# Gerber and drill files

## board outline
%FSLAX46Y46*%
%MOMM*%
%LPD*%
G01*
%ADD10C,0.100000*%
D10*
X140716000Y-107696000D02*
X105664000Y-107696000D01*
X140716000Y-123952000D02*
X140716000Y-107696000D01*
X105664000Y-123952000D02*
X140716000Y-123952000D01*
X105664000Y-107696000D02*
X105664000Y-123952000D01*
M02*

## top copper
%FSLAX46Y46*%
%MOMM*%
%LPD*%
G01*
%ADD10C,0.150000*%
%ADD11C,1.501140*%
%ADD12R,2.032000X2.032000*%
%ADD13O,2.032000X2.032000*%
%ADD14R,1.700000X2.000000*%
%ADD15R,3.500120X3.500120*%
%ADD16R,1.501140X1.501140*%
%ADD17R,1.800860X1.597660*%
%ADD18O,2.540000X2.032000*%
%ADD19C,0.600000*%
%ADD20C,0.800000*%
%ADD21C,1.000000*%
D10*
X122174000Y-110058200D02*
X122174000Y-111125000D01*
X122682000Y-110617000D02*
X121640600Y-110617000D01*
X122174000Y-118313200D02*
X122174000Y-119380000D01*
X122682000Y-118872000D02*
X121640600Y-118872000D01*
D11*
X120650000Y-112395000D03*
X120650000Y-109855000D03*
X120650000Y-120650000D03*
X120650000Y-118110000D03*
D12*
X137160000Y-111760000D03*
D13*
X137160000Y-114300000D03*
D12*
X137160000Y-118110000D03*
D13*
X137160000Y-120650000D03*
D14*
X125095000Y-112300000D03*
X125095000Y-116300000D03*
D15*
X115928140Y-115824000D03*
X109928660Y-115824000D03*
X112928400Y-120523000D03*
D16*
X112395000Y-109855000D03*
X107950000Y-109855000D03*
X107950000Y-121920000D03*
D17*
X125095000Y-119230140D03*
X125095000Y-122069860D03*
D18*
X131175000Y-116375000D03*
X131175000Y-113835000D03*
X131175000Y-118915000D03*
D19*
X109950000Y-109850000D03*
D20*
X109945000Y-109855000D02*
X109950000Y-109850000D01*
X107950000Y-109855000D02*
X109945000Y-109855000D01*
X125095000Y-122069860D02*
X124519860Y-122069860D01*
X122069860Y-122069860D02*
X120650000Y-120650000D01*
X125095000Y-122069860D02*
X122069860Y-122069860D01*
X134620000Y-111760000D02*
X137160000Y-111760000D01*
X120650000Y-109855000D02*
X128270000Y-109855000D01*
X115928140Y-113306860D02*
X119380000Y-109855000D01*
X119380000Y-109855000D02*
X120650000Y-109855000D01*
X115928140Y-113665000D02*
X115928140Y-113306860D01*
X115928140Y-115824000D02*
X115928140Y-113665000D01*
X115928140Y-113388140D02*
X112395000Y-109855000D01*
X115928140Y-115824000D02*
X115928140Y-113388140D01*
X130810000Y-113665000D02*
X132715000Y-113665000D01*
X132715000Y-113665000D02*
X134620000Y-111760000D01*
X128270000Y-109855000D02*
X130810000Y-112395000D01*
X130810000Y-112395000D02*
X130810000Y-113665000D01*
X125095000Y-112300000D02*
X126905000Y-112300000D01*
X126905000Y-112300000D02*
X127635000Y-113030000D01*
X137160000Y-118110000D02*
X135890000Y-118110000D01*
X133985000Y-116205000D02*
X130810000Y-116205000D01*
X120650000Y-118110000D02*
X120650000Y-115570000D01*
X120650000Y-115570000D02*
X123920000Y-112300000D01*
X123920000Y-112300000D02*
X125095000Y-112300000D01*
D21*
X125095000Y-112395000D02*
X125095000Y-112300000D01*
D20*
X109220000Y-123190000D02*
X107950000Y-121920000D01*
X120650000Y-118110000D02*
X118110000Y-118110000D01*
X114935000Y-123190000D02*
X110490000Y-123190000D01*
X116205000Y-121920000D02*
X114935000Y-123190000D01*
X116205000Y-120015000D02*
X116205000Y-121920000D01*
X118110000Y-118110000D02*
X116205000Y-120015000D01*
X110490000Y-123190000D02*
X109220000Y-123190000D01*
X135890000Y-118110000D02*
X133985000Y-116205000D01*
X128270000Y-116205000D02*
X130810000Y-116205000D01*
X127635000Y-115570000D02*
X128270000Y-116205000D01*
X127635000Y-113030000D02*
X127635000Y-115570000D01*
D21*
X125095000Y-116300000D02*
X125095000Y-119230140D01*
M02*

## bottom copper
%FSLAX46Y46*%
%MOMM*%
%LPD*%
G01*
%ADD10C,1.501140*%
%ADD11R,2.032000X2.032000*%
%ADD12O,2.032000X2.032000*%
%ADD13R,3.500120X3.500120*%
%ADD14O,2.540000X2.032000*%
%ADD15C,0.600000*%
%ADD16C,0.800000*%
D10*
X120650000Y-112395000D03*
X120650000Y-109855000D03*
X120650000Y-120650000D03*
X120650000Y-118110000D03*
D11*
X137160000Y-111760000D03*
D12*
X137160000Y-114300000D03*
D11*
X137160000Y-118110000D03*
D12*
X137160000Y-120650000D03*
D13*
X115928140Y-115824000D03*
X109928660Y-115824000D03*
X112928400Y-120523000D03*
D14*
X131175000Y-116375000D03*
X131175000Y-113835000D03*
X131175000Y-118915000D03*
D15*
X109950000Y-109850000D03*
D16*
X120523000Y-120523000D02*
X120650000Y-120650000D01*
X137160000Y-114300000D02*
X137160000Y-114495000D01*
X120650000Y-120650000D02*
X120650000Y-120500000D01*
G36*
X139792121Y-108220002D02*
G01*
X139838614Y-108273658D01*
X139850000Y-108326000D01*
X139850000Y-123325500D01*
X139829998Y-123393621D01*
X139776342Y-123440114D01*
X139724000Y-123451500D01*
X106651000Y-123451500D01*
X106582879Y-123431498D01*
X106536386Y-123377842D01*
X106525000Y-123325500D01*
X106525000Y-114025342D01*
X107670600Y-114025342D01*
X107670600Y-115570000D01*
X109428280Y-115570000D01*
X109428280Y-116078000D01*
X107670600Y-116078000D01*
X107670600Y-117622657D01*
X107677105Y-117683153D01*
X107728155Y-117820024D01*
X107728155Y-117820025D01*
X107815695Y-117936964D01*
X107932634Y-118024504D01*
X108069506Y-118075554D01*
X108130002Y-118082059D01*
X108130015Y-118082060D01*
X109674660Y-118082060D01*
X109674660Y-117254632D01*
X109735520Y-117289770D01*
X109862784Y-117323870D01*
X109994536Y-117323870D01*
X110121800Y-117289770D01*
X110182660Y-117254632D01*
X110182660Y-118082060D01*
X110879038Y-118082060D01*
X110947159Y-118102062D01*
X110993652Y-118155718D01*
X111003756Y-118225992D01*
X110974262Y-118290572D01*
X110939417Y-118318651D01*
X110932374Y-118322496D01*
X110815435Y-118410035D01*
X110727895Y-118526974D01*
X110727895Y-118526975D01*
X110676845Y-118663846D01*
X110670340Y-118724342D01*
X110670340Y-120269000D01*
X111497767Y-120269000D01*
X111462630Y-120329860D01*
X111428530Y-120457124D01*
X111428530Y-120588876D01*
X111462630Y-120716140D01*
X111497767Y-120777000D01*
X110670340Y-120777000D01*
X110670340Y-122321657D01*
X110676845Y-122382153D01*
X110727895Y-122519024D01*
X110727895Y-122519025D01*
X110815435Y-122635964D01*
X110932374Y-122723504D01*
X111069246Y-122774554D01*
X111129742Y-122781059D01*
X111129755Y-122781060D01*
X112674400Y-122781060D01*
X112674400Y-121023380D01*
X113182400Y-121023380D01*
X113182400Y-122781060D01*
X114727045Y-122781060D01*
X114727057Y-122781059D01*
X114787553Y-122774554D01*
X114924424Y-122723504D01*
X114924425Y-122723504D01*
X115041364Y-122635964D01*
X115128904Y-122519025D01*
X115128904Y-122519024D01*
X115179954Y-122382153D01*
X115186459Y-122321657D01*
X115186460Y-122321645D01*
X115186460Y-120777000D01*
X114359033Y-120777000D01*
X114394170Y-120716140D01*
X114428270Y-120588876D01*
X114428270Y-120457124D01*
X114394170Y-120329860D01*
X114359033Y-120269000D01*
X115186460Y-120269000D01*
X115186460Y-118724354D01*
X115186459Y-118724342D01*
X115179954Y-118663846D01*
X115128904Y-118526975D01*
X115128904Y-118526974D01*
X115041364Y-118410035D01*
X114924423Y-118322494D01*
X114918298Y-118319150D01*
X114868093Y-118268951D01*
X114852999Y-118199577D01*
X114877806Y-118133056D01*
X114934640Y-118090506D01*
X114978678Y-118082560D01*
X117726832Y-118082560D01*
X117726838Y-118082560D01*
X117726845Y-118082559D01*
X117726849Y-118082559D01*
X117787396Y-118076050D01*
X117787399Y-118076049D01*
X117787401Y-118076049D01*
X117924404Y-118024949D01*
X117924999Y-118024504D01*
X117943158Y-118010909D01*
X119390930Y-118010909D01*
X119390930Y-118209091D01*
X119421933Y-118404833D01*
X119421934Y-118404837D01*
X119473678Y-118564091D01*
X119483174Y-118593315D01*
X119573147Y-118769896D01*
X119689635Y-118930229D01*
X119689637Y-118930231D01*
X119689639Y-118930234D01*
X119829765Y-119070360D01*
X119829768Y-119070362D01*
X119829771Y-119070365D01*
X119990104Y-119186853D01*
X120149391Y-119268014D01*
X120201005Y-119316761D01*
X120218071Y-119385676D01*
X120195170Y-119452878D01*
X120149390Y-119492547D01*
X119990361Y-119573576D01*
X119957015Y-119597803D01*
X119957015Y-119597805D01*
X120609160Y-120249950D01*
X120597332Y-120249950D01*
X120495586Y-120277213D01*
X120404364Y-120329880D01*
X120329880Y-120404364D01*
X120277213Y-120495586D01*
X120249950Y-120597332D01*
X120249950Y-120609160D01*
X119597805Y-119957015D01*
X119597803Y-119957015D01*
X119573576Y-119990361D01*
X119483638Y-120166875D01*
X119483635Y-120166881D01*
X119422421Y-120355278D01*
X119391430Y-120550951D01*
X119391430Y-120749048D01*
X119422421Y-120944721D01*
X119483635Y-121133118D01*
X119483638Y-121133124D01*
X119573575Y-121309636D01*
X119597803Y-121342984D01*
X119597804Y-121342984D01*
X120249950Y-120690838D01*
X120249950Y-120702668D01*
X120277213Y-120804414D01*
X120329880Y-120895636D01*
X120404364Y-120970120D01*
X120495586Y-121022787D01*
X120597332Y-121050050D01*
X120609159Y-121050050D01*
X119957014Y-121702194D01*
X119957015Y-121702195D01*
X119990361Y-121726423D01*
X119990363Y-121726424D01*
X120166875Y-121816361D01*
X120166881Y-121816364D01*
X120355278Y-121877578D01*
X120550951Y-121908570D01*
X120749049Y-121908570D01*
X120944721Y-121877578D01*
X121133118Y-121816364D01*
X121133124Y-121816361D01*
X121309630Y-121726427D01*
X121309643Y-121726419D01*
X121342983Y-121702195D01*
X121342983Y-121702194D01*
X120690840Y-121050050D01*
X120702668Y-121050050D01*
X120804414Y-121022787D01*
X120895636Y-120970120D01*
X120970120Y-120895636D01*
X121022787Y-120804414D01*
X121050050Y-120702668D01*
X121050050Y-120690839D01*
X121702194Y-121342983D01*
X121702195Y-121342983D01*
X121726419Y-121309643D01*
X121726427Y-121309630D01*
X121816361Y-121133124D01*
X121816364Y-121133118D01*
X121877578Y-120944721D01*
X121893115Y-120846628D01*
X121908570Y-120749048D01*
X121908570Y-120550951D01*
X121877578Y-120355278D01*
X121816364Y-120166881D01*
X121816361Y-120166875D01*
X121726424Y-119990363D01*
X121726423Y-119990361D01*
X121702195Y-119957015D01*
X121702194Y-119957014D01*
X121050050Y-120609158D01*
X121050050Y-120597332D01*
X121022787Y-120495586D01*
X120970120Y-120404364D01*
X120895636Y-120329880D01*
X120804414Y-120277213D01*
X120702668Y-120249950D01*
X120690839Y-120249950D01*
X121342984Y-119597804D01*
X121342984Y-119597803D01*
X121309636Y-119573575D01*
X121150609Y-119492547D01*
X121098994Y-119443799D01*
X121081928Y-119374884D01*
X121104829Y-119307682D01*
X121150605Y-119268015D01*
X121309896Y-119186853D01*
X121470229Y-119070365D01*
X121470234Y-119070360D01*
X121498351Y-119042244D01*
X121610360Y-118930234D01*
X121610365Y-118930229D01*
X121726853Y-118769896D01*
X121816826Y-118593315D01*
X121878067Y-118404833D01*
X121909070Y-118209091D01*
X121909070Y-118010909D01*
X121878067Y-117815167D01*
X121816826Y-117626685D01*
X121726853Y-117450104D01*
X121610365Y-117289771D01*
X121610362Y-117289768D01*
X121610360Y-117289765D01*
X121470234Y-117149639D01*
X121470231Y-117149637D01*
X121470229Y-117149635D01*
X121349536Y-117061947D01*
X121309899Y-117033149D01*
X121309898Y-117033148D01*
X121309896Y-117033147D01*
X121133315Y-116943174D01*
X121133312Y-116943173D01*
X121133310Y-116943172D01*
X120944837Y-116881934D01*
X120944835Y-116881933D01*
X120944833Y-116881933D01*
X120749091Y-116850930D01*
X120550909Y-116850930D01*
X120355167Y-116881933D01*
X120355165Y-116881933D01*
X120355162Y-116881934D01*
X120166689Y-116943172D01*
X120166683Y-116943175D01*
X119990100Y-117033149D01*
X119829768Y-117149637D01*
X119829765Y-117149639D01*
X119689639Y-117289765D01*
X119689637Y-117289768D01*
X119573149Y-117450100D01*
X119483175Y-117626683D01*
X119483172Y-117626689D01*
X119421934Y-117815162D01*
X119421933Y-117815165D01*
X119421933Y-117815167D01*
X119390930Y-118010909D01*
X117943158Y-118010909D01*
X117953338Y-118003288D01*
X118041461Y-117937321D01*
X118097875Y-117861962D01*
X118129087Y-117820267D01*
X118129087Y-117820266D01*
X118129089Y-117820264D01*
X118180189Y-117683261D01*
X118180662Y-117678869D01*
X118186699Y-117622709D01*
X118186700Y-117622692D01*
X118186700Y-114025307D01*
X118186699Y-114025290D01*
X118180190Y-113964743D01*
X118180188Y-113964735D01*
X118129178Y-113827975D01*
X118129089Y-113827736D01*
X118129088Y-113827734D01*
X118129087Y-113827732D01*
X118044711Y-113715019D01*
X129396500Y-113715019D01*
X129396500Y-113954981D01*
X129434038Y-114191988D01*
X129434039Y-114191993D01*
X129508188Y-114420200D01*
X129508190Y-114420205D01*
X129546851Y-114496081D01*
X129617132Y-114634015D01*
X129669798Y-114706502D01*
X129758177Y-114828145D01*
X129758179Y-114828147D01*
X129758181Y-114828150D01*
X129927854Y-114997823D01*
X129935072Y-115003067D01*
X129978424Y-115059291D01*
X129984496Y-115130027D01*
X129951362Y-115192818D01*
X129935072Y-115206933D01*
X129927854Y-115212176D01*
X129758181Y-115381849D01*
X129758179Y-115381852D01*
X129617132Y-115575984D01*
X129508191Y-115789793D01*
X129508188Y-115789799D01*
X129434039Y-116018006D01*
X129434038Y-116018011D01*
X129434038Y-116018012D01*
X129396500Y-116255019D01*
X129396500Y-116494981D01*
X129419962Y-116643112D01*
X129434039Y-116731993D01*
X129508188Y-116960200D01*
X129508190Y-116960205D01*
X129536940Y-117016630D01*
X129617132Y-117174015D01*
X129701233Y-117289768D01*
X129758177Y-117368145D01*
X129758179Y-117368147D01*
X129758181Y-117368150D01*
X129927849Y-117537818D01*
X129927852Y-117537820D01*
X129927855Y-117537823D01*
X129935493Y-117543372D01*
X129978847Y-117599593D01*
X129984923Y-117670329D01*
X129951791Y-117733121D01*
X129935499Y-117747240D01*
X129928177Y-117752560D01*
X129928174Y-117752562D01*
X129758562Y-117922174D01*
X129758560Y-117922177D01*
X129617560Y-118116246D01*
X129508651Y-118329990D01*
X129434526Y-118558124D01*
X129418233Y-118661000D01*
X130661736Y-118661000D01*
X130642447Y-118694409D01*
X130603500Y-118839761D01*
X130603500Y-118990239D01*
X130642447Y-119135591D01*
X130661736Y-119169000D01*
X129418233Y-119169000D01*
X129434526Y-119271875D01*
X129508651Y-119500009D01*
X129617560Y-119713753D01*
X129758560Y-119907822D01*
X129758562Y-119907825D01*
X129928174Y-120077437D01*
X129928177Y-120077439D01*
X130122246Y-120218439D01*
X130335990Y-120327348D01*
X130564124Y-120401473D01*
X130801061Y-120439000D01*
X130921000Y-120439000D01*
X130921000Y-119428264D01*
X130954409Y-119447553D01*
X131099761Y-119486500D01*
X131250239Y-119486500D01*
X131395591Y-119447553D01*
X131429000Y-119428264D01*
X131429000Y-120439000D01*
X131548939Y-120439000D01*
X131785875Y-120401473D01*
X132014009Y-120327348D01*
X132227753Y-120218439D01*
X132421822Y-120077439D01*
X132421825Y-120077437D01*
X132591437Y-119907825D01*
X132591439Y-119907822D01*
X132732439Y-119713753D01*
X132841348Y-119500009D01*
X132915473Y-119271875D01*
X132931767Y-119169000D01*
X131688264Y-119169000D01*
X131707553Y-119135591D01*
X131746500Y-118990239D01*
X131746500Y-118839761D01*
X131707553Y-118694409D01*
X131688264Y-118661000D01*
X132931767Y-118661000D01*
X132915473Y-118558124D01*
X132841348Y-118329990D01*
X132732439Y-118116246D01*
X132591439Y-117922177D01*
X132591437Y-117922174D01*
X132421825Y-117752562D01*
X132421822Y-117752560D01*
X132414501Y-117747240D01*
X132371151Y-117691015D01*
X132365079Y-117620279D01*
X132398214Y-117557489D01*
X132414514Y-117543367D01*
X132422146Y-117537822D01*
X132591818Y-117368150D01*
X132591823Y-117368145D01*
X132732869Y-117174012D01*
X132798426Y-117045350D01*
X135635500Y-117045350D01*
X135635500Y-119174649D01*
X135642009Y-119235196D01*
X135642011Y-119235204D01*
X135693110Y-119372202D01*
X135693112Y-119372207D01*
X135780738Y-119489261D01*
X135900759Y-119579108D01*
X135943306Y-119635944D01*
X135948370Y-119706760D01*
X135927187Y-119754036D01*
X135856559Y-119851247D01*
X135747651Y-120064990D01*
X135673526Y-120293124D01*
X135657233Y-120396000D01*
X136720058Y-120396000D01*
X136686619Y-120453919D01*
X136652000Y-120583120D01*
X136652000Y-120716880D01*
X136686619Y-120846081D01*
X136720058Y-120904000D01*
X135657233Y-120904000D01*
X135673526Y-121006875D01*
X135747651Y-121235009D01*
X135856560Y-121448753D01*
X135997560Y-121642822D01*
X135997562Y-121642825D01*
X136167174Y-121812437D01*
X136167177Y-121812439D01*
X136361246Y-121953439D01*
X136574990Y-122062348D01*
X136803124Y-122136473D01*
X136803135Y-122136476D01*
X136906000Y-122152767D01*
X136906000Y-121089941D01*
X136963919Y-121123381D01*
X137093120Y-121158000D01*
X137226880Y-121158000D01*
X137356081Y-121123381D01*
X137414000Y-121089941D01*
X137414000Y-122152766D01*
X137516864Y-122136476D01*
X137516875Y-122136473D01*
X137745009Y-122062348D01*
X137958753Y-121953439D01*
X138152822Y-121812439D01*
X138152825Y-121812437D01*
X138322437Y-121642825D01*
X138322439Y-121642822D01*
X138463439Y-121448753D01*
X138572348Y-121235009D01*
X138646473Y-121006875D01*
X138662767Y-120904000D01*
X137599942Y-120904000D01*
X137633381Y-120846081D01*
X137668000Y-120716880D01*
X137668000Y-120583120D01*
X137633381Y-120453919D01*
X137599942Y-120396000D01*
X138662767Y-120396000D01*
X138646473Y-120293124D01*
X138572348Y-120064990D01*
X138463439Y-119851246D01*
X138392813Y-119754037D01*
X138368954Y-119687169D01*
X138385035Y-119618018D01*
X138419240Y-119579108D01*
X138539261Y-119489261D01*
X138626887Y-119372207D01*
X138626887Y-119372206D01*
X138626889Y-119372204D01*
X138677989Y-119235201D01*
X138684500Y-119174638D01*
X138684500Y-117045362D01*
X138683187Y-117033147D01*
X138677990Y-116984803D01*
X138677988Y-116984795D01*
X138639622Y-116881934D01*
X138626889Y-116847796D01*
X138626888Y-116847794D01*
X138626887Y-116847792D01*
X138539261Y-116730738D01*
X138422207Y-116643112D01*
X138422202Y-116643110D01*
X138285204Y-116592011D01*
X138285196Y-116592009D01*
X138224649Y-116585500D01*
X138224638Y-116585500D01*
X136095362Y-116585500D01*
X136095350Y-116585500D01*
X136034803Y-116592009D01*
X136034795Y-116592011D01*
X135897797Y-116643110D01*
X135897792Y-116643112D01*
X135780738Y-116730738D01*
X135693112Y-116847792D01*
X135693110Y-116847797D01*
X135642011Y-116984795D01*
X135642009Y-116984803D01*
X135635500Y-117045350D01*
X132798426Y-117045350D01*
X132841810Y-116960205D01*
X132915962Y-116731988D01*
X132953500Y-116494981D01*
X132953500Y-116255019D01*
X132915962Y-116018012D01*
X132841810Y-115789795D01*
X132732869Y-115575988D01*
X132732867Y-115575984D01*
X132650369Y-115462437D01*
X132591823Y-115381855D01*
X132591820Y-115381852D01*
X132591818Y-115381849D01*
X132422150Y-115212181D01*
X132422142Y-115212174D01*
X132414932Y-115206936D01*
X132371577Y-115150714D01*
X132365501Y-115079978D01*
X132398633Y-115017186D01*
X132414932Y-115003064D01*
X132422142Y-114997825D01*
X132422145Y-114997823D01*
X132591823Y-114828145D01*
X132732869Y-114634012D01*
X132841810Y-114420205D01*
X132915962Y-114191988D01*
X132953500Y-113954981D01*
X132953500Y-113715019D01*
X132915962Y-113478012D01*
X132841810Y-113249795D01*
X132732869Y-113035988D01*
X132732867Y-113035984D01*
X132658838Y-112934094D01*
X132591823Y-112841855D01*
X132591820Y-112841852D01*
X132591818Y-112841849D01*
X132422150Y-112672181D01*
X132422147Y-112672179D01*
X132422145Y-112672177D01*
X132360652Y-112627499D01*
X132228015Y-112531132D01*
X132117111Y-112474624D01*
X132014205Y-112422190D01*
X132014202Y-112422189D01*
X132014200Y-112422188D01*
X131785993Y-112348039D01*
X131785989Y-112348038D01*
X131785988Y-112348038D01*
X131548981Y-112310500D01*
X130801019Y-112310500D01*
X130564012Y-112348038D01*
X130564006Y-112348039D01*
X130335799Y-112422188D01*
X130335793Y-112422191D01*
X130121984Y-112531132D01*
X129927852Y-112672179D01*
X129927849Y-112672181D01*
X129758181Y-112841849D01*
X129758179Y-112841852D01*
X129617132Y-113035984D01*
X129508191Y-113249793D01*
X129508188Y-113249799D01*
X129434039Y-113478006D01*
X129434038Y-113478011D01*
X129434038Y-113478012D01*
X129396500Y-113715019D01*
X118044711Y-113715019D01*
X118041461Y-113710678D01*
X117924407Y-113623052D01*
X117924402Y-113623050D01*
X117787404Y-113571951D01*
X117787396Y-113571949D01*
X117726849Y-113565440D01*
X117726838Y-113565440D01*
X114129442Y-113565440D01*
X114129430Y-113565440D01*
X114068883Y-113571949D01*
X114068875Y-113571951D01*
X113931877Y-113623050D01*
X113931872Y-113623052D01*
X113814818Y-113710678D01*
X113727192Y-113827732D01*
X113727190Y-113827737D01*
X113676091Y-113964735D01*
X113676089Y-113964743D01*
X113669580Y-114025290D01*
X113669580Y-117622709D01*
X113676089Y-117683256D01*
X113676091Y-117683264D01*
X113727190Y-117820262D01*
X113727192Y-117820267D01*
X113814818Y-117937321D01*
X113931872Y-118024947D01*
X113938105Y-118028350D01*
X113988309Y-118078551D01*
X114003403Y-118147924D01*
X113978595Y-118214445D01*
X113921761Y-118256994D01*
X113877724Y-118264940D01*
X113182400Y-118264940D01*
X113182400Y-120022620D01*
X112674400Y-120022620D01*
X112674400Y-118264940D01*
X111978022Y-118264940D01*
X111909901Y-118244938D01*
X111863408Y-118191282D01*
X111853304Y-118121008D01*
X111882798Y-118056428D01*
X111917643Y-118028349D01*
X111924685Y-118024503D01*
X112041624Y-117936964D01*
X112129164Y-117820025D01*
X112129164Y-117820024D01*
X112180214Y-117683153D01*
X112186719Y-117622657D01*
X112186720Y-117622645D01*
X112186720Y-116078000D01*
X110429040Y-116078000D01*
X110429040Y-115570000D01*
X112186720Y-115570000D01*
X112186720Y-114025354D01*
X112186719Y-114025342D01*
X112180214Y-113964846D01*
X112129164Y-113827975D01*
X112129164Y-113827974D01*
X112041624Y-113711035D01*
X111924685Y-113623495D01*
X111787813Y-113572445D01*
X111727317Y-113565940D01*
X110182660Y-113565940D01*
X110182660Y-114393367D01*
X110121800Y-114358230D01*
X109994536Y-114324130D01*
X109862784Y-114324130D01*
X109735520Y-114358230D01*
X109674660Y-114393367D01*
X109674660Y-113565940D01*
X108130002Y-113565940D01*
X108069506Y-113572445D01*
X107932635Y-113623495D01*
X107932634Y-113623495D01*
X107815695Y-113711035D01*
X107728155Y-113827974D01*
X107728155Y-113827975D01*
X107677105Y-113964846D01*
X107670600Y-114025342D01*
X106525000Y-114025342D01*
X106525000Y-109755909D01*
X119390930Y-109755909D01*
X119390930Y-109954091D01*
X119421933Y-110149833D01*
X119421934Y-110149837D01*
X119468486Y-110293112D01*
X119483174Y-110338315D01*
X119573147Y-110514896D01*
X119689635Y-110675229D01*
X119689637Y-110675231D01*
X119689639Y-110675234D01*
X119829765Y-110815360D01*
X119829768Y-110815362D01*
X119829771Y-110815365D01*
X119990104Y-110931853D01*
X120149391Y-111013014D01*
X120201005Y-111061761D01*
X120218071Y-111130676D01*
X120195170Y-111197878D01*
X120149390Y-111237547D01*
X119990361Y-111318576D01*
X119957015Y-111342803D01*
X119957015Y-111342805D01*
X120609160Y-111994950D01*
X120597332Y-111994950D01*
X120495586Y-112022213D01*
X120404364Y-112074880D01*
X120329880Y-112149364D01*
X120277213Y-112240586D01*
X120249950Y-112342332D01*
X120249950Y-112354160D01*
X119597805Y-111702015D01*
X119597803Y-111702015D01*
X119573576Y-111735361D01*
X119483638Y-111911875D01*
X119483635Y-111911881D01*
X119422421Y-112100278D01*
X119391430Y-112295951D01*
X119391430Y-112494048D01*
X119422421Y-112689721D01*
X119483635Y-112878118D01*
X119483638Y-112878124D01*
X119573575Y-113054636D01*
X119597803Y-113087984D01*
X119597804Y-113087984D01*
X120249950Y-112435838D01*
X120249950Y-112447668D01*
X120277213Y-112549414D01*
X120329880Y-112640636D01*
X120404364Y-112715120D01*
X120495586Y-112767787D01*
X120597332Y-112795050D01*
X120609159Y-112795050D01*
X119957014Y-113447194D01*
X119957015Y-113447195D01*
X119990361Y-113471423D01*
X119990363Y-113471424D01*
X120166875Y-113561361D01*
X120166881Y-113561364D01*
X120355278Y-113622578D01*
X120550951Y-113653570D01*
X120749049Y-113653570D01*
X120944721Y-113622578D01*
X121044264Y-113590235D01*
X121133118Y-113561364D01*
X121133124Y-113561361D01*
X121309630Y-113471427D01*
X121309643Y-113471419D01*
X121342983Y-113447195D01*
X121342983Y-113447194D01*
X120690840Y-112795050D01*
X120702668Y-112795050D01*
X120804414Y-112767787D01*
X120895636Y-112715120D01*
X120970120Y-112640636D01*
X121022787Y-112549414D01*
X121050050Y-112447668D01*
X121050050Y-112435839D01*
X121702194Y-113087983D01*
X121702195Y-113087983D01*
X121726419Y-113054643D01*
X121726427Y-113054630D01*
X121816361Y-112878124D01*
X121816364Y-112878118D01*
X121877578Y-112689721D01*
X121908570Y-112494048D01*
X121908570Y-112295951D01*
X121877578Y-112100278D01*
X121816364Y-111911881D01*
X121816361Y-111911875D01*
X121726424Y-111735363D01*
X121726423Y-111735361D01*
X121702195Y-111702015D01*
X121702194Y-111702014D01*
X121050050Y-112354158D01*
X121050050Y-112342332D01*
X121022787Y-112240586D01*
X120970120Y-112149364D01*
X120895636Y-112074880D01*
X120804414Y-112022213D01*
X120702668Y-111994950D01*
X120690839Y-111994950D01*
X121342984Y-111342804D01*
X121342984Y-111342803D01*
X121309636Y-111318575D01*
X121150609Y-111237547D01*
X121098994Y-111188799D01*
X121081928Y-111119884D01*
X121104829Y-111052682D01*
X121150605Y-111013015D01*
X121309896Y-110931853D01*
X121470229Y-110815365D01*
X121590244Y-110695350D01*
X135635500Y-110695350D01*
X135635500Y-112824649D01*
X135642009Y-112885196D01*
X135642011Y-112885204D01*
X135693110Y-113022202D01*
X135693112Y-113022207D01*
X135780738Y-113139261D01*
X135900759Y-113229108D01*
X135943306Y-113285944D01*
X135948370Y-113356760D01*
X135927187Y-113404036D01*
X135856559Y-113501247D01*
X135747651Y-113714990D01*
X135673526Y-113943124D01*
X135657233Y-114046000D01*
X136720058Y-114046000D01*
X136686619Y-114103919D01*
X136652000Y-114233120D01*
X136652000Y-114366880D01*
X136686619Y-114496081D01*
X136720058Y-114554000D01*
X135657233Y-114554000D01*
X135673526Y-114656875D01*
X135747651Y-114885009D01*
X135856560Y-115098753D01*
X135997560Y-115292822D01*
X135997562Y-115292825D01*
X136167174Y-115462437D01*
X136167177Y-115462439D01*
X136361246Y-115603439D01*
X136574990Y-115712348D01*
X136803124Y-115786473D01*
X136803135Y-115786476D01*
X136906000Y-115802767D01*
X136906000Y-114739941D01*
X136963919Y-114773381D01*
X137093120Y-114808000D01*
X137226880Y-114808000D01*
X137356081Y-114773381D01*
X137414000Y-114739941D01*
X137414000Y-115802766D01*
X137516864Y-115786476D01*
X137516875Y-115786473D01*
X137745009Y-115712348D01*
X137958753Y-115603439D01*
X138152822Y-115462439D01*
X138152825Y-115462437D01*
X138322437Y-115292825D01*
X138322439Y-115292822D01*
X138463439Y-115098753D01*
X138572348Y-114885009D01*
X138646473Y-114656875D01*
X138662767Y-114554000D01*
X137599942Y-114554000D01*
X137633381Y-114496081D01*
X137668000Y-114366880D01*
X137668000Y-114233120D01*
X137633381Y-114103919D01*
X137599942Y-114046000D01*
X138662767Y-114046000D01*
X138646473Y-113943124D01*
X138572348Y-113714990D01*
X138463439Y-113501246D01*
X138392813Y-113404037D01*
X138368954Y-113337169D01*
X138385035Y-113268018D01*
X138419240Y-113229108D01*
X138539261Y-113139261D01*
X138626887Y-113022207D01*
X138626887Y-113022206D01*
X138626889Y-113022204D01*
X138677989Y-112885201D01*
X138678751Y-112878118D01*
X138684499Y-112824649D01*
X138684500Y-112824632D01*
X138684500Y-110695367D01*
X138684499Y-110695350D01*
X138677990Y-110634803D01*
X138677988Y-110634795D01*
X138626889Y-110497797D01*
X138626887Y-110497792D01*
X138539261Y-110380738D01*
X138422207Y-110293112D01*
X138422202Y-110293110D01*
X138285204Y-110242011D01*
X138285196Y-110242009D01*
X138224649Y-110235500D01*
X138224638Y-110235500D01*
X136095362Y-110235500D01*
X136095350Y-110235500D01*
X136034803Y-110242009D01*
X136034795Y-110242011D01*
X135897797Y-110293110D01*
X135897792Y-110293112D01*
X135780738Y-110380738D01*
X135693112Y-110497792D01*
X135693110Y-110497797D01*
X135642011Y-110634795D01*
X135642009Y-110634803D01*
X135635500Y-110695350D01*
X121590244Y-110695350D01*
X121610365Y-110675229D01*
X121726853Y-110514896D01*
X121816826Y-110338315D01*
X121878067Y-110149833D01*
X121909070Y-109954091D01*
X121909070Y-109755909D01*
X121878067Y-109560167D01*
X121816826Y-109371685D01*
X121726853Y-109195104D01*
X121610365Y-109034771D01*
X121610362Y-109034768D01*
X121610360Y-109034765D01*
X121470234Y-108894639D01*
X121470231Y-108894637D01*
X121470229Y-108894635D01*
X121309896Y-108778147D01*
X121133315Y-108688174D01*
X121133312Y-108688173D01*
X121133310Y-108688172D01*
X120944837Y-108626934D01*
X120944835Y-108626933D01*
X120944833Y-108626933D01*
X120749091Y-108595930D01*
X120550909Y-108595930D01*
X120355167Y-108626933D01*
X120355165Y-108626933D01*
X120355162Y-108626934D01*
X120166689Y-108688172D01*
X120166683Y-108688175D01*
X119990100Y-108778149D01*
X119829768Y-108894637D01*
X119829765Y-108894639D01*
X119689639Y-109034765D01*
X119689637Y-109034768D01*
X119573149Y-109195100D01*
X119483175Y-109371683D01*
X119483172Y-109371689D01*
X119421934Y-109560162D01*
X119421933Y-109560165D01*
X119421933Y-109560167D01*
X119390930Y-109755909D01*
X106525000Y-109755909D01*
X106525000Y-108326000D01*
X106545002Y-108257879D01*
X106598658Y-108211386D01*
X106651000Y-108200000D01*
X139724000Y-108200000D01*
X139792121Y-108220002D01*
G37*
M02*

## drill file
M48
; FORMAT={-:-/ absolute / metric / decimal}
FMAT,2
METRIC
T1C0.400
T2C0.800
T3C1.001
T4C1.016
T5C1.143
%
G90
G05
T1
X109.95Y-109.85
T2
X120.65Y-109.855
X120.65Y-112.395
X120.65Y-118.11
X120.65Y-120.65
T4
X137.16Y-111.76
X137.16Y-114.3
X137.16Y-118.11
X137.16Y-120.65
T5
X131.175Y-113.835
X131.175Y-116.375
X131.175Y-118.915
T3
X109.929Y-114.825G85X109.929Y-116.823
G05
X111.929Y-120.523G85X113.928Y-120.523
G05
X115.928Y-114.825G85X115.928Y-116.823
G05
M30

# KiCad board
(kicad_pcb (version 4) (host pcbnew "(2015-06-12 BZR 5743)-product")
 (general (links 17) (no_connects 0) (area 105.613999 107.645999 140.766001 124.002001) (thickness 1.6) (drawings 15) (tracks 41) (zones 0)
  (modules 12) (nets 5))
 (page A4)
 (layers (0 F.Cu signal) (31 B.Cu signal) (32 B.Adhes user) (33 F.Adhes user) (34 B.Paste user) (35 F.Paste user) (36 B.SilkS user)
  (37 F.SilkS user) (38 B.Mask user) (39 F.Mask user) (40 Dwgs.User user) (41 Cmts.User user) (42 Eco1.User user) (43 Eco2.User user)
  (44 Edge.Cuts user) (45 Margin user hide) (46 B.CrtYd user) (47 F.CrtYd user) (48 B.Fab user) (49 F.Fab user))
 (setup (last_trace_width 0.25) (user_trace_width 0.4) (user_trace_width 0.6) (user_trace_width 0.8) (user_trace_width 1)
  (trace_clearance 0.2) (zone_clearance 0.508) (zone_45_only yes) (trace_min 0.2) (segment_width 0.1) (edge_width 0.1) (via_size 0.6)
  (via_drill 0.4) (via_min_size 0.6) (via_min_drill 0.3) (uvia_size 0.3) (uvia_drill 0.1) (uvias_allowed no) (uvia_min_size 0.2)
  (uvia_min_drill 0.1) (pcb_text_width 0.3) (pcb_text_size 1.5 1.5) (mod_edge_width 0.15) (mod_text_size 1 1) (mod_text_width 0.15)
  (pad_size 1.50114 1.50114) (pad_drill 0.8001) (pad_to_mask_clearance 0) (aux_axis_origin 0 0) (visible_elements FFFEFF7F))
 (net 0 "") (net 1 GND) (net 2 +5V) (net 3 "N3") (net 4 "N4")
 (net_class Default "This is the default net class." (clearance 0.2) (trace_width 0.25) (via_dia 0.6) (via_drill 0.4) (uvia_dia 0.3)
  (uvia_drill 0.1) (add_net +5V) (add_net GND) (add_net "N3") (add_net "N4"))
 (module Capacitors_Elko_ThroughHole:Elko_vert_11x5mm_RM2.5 (layer F.Cu) (at 120.65 109.855 270)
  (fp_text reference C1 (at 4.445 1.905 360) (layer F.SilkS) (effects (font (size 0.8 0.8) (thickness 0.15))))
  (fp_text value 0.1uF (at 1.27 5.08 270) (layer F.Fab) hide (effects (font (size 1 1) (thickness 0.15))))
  (fp_line (start 0.2032 -1.524) (end 1.27 -1.524) (layer F.Cu) (width 0.15))
  (fp_line (start 0.762 -2.032) (end 0.762 -0.9906) (layer F.Cu) (width 0.15))
  (pad 2 thru_hole circle (at 2.54 0 270) (size 1.50114 1.50114) (drill 0.8001) (layers *.Cu *.Mask F.SilkS) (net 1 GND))
  (pad 1 thru_hole circle (at 0 0 270) (size 1.50114 1.50114) (drill 0.8001) (layers *.Cu *.Mask F.SilkS) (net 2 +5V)))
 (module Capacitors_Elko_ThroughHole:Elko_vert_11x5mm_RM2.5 (layer F.Cu) (at 120.65 118.11 270)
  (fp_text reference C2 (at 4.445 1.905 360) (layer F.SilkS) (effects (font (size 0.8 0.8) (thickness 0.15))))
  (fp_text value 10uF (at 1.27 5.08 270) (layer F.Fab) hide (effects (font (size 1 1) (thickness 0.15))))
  (fp_line (start 0.2032 -1.524) (end 1.27 -1.524) (layer F.Cu) (width 0.15))
  (fp_line (start 0.762 -2.032) (end 0.762 -0.9906) (layer F.Cu) (width 0.15))
  (pad 2 thru_hole circle (at 2.54 0 270) (size 1.50114 1.50114) (drill 0.8001) (layers *.Cu *.Mask F.SilkS) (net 1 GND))
  (pad 1 thru_hole circle (at 0 0 270) (size 1.50114 1.50114) (drill 0.8001) (layers *.Cu *.Mask F.SilkS) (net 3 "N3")))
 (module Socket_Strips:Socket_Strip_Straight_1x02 (layer F.Cu) (at 137.16 111.76 270)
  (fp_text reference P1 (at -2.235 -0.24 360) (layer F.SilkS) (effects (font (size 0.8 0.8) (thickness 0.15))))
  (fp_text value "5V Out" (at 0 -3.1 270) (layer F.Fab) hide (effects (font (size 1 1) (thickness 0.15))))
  (pad 1 thru_hole rect (at 0 0 270) (size 2.032 2.032) (drill 1.016) (layers *.Cu *.Mask F.SilkS) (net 2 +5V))
  (pad 2 thru_hole oval (at 2.54 0 270) (size 2.032 2.032) (drill 1.016) (layers *.Cu *.Mask F.SilkS) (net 1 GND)))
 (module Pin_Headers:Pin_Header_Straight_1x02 (layer B.Cu) (at 137.16 118.11 180)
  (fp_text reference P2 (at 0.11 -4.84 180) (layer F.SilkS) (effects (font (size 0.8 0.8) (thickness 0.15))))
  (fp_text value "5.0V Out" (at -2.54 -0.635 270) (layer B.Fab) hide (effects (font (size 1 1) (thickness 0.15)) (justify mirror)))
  (pad 1 thru_hole rect (at 0 0 180) (size 2.032 2.032) (drill 1.016) (layers *.Cu *.Mask B.SilkS) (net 3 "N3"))
  (pad 2 thru_hole oval (at 0 -2.54 180) (size 2.032 2.032) (drill 1.016) (layers *.Cu *.Mask B.SilkS) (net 1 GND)))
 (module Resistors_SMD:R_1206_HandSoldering (layer F.Cu) (at 125.095 114.3 270)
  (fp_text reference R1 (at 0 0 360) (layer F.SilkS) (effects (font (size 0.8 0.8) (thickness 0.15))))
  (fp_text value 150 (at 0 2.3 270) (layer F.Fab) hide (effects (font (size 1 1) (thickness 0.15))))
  (pad 1 smd rect (at -2 0 270) (size 2 1.7) (layers F.Cu F.Paste F.Mask) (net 3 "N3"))
  (pad 2 smd rect (at 2 0 270) (size 2 1.7) (layers F.Cu F.Paste F.Mask) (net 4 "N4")))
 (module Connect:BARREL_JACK (layer F.Cu) (at 109.728 115.824)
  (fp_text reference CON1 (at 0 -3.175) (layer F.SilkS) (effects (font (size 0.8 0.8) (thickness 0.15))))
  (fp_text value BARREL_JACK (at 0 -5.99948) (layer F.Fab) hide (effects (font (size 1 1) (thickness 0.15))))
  (pad 1 thru_hole rect (at 6.20014 0) (size 3.50012 3.50012) (drill oval 1.00076 2.99974) (layers *.Cu *.Mask F.SilkS) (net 2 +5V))
  (pad 2 thru_hole rect (at 0.20066 0) (size 3.50012 3.50012) (drill oval 1.00076 2.99974) (layers *.Cu *.Mask F.SilkS) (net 1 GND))
  (pad 3 thru_hole rect (at 3.2004 4.699) (size 3.50012 3.50012) (drill oval 2.99974 1.00076) (layers *.Cu *.Mask F.SilkS) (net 1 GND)))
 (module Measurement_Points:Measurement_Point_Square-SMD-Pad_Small (layer F.Cu) (at 112.395 109.855)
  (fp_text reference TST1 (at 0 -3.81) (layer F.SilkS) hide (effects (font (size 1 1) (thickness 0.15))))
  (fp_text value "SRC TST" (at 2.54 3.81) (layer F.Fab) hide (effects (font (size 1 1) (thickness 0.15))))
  (pad 1 smd rect (at 0 0) (size 1.50114 1.50114) (layers F.Cu F.Paste F.Mask) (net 2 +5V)))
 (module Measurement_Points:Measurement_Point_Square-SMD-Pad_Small (layer F.Cu) (at 107.95 109.855)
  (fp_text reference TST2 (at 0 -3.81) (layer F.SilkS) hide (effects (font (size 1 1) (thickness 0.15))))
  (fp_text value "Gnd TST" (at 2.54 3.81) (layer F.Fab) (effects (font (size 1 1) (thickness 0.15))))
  (pad 1 smd rect (at 0 0) (size 1.50114 1.50114) (layers F.Cu F.Paste F.Mask) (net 1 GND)))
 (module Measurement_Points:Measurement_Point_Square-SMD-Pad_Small (layer F.Cu) (at 107.95 121.92)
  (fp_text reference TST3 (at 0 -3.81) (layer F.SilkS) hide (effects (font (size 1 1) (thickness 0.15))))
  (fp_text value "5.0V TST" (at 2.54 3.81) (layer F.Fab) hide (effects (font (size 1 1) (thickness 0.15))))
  (pad 1 smd rect (at 0 0) (size 1.50114 1.50114) (layers F.Cu F.Paste F.Mask) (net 3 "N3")))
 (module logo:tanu (layer B.Cu) (at 125.3 115.75 90)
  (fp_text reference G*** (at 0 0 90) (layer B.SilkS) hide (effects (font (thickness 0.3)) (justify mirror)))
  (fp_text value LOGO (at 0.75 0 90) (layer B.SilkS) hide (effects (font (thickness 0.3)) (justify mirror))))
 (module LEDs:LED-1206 (layer F.Cu) (at 125.095 120.65 90)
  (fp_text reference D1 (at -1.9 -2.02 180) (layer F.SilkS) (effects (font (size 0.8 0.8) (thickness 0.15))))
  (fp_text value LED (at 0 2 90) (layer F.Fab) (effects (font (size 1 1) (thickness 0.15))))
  (pad 2 smd rect (at 1.41986 0 270) (size 1.59766 1.80086) (layers F.Cu F.Paste F.Mask) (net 4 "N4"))
  (pad 1 smd rect (at -1.41986 0 270) (size 1.59766 1.80086) (layers F.Cu F.Paste F.Mask) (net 1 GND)))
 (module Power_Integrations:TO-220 (layer F.Cu) (at 131.175 116.375 90)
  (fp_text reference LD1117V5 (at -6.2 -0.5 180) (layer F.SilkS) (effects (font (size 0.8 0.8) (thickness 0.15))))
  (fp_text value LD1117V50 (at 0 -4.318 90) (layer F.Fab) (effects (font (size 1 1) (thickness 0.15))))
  (pad 2 thru_hole oval (at 0 0 90) (size 2.032 2.54) (drill 1.143) (layers *.Cu *.Mask F.SilkS) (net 3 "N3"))
  (pad 3 thru_hole oval (at 2.54 0 90) (size 2.032 2.54) (drill 1.143) (layers *.Cu *.Mask F.SilkS) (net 2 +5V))
  (pad 1 thru_hole oval (at -2.54 0 90) (size 2.032 2.54) (drill 1.143) (layers *.Cu *.Mask F.SilkS) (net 1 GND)))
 (gr_line (start 140.716 107.696) (end 105.664 107.696) (angle 90) (layer Edge.Cuts) (width 0.1))
 (gr_line (start 140.716 123.952) (end 140.716 107.696) (angle 90) (layer Edge.Cuts) (width 0.1))
 (gr_line (start 105.664 123.952) (end 140.716 123.952) (angle 90) (layer Edge.Cuts) (width 0.1))
 (gr_line (start 105.664 107.696) (end 105.664 123.952) (angle 90) (layer Edge.Cuts) (width 0.1))
 (segment (start 120.523 120.523) (end 120.65 120.65) (width 0.8) (layer B.Cu) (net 1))
 (segment (start 137.16 114.3) (end 137.16 114.495) (width 0.8) (layer B.Cu) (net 1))
 (segment (start 120.65 120.65) (end 120.65 120.5) (width 0.8) (layer B.Cu) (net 1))
 (segment (start 109.945 109.855) (end 109.95 109.85) (width 0.8) (layer F.Cu) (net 1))
 (via (at 109.95 109.85) (size 0.6) (layers F.Cu B.Cu) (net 1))
 (segment (start 107.95 109.855) (end 109.945 109.855) (width 0.8) (layer F.Cu) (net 1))
 (segment (start 125.095 122.06986) (end 124.51986 122.06986) (width 0.8) (layer F.Cu) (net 1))
 (segment (start 122.06986 122.06986) (end 120.65 120.65) (width 0.8) (layer F.Cu) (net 1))
 (segment (start 125.095 122.06986) (end 122.06986 122.06986) (width 0.8) (layer F.Cu) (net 1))
 (segment (start 134.62 111.76) (end 137.16 111.76) (width 0.8) (layer F.Cu) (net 2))
 (segment (start 120.65 109.855) (end 128.27 109.855) (width 0.8) (layer F.Cu) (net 2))
 (segment (start 115.92814 113.30686) (end 119.38 109.855) (width 0.8) (layer F.Cu) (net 2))
 (segment (start 119.38 109.855) (end 120.65 109.855) (width 0.8) (layer F.Cu) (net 2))
 (segment (start 115.92814 113.665) (end 115.92814 113.30686) (width 0.8) (layer F.Cu) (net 2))
 (segment (start 115.92814 115.824) (end 115.92814 113.665) (width 0.8) (layer F.Cu) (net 2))
 (segment (start 115.92814 113.38814) (end 112.395 109.855) (width 0.8) (layer F.Cu) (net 2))
 (segment (start 115.92814 115.824) (end 115.92814 113.38814) (width 0.8) (layer F.Cu) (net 2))
 (segment (start 130.81 113.665) (end 132.715 113.665) (width 0.8) (layer F.Cu) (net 2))
 (segment (start 132.715 113.665) (end 134.62 111.76) (width 0.8) (layer F.Cu) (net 2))
 (segment (start 128.27 109.855) (end 130.81 112.395) (width 0.8) (layer F.Cu) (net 2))
 (segment (start 130.81 112.395) (end 130.81 113.665) (width 0.8) (layer F.Cu) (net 2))
 (segment (start 125.095 112.3) (end 126.905 112.3) (width 0.8) (layer F.Cu) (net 3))
 (segment (start 126.905 112.3) (end 127.635 113.03) (width 0.8) (layer F.Cu) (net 3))
 (segment (start 137.16 118.11) (end 135.89 118.11) (width 0.8) (layer F.Cu) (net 3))
 (segment (start 133.985 116.205) (end 130.81 116.205) (width 0.8) (layer F.Cu) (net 3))
 (segment (start 120.65 118.11) (end 120.65 115.57) (width 0.8) (layer F.Cu) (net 3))
 (segment (start 120.65 115.57) (end 123.92 112.3) (width 0.8) (layer F.Cu) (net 3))
 (segment (start 123.92 112.3) (end 125.095 112.3) (width 0.8) (layer F.Cu) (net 3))
 (segment (start 125.095 112.395) (end 125.095 112.3) (width 1) (layer F.Cu) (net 3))
 (segment (start 109.22 123.19) (end 107.95 121.92) (width 0.8) (layer F.Cu) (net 3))
 (segment (start 120.65 118.11) (end 118.11 118.11) (width 0.8) (layer F.Cu) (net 3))
 (segment (start 114.935 123.19) (end 110.49 123.19) (width 0.8) (layer F.Cu) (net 3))
 (segment (start 116.205 121.92) (end 114.935 123.19) (width 0.8) (layer F.Cu) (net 3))
 (segment (start 116.205 120.015) (end 116.205 121.92) (width 0.8) (layer F.Cu) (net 3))
 (segment (start 118.11 118.11) (end 116.205 120.015) (width 0.8) (layer F.Cu) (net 3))
 (segment (start 110.49 123.19) (end 109.22 123.19) (width 0.8) (layer F.Cu) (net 3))
 (segment (start 135.89 118.11) (end 133.985 116.205) (width 0.8) (layer F.Cu) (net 3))
 (segment (start 128.27 116.205) (end 130.81 116.205) (width 0.8) (layer F.Cu) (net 3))
 (segment (start 127.635 115.57) (end 128.27 116.205) (width 0.8) (layer F.Cu) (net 3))
 (segment (start 127.635 113.03) (end 127.635 115.57) (width 0.8) (layer F.Cu) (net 3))
 (segment (start 125.095 116.3) (end 125.095 119.23014) (width 1) (layer F.Cu) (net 4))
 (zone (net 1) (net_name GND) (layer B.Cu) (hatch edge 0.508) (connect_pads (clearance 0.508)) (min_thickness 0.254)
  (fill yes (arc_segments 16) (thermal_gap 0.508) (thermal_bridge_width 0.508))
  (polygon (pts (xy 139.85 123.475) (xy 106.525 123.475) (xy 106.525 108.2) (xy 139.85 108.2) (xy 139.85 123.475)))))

